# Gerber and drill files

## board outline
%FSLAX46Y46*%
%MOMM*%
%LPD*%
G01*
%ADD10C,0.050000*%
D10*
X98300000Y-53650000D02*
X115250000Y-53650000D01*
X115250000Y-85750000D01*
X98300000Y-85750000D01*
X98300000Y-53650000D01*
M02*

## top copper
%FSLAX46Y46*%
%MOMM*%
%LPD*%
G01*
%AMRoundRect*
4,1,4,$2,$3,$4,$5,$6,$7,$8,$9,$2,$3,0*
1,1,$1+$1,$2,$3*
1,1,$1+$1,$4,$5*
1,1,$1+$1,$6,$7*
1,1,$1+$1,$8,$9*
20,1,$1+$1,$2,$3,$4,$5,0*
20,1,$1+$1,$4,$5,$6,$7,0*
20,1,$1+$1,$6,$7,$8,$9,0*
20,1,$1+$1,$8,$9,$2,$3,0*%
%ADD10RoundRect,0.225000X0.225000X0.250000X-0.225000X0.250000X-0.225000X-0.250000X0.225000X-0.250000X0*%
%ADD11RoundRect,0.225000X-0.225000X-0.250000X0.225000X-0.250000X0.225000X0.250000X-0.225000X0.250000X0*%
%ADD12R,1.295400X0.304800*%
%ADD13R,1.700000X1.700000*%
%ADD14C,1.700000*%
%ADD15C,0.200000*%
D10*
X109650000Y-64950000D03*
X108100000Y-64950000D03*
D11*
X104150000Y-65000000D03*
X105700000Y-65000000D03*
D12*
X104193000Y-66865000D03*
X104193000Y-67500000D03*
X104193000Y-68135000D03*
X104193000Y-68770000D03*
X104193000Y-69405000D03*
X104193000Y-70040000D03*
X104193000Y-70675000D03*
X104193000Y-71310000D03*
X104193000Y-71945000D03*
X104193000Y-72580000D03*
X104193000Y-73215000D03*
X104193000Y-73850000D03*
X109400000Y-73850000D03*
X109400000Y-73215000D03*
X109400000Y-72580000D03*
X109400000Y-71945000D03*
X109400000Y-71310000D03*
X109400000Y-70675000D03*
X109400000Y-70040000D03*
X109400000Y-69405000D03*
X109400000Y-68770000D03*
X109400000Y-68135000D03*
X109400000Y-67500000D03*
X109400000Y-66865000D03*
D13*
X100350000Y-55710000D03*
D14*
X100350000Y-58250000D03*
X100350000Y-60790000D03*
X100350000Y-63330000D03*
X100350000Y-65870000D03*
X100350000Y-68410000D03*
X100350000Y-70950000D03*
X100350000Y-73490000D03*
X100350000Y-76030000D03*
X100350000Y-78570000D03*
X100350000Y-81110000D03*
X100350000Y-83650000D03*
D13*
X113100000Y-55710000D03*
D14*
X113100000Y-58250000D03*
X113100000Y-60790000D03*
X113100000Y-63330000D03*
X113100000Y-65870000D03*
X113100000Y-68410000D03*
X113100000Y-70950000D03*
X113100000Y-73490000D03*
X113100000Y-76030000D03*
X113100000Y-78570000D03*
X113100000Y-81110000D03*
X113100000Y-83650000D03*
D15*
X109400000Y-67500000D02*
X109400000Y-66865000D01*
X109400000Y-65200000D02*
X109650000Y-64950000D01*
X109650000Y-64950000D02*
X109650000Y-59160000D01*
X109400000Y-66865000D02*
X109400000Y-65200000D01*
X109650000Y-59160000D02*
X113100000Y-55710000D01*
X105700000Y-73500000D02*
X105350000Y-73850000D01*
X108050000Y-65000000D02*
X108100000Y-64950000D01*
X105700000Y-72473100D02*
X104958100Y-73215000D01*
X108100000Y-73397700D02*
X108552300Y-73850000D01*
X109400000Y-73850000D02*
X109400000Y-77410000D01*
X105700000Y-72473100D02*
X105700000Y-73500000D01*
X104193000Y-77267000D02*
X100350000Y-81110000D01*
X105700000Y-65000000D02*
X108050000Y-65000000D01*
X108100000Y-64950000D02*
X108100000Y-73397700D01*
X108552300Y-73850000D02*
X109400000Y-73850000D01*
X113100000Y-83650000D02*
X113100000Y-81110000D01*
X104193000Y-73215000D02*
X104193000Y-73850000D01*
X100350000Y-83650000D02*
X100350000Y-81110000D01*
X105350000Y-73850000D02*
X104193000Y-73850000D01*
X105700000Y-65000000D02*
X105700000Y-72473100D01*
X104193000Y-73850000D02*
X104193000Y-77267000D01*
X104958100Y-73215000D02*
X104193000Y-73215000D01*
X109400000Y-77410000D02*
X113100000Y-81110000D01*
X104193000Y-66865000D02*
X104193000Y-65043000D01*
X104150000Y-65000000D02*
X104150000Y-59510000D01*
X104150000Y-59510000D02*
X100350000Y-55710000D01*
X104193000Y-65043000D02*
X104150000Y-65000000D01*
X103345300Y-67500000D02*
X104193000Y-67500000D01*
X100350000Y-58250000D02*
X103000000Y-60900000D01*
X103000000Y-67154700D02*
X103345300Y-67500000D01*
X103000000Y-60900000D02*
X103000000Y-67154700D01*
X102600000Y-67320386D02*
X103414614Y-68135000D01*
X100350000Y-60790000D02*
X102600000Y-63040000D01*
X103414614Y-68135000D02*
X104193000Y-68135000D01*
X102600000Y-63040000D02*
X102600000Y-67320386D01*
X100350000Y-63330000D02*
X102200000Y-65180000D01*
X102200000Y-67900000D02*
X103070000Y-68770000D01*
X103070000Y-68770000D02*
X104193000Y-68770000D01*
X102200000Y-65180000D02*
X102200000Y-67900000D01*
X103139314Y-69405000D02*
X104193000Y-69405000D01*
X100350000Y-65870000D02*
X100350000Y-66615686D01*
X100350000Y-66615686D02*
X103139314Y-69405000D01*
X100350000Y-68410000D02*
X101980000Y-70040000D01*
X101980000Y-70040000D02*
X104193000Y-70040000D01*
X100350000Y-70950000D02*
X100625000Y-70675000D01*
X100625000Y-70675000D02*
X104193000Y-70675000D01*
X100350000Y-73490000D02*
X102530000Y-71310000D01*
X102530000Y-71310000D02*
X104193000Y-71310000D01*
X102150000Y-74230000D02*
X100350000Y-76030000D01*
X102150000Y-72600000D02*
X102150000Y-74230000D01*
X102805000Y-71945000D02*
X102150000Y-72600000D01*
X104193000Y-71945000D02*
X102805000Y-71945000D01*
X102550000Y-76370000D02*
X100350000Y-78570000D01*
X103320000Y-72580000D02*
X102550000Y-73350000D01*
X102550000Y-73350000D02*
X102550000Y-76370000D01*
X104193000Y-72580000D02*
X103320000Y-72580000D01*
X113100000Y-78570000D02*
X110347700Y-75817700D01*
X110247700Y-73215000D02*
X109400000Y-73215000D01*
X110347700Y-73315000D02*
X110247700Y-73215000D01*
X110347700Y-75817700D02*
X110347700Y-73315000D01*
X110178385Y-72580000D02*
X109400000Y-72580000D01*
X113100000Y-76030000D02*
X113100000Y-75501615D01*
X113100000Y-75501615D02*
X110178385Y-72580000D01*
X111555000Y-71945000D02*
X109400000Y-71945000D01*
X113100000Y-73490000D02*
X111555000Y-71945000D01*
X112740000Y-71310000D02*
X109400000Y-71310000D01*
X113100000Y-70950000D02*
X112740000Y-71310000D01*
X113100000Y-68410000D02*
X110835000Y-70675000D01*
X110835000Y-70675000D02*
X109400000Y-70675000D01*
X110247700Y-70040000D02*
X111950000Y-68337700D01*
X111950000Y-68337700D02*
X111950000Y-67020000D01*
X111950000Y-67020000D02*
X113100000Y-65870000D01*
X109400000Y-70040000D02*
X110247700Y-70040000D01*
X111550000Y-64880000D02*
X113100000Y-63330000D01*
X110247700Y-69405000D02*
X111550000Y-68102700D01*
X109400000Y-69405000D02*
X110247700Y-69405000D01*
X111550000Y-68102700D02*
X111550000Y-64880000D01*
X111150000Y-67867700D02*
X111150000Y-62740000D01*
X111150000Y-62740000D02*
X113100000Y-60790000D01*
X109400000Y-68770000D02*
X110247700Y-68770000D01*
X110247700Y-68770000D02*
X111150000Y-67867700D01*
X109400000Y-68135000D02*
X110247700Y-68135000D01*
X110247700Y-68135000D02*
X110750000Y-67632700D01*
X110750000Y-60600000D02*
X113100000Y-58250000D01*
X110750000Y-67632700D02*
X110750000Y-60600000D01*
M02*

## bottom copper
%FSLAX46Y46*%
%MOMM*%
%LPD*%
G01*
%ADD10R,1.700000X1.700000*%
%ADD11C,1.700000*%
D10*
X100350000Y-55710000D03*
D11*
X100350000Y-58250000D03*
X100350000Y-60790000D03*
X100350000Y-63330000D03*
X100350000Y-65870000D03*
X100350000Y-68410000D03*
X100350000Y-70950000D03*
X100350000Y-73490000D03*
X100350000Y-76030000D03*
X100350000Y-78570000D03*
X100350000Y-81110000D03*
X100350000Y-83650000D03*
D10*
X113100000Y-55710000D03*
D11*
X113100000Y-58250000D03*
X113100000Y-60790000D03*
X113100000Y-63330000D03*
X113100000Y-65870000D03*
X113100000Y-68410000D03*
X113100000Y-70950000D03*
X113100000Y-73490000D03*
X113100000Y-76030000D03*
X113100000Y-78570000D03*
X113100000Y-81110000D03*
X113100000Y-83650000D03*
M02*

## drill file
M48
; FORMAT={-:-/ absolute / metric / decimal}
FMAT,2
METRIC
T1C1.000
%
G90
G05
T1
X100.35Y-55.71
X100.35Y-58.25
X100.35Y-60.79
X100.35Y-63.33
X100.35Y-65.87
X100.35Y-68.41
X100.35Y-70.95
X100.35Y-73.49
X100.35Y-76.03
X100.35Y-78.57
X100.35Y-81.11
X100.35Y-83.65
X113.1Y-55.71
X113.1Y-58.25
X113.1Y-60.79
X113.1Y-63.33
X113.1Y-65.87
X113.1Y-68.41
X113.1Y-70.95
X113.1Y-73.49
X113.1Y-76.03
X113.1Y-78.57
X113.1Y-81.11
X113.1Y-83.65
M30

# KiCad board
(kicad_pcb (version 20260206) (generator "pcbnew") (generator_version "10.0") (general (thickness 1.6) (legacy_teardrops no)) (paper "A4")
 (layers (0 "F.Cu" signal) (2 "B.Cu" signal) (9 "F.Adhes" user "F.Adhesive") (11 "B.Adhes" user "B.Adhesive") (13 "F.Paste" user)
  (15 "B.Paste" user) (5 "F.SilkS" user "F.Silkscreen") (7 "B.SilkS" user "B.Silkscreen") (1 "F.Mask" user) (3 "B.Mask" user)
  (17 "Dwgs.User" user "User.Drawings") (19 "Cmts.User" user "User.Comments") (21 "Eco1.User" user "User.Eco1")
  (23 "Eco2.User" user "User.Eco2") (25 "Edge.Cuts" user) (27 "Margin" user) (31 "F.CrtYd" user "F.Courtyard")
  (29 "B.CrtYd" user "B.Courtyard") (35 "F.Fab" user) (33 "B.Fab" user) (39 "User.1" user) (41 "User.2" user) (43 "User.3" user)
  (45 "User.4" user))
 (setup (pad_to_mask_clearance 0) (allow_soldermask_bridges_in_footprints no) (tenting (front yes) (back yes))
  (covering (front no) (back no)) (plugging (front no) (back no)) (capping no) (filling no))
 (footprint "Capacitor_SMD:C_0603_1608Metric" (layer "F.Cu") (at 108.875 64.95 180)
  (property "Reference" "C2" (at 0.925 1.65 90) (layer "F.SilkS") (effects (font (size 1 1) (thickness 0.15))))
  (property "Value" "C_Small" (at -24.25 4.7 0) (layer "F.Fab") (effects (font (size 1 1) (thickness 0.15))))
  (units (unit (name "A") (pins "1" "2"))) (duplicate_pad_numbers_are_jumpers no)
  (pad "1" smd roundrect (at -0.775 0 180) (size 0.9 0.95) (layers "F.Cu" "F.Mask" "F.Paste") (roundrect_rratio 0.25) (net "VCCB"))
  (pad "2" smd roundrect (at 0.775 0 180) (size 0.9 0.95) (layers "F.Cu" "F.Mask" "F.Paste") (roundrect_rratio 0.25) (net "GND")))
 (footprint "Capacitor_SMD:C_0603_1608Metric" (layer "F.Cu") (at 104.925 65)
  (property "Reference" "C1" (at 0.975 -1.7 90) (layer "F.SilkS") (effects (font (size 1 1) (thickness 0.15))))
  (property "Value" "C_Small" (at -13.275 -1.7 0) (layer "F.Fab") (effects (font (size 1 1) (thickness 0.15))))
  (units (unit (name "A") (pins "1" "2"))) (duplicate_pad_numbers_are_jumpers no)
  (pad "1" smd roundrect (at -0.775 0) (size 0.9 0.95) (layers "F.Cu" "F.Mask" "F.Paste") (roundrect_rratio 0.25) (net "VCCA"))
  (pad "2" smd roundrect (at 0.775 0) (size 0.9 0.95) (layers "F.Cu" "F.Mask" "F.Paste") (roundrect_rratio 0.25) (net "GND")))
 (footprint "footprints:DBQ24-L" (layer "F.Cu") (at 106.7965 70.3575)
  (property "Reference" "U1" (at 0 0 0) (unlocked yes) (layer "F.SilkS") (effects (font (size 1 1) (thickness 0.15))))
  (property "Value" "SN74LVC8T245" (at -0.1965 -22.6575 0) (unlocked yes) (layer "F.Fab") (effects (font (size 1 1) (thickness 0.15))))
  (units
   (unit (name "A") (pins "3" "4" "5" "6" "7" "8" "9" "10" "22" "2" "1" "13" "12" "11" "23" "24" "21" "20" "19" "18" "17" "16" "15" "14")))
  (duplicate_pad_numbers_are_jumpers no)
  (pad "1" smd rect (at -2.6035 -3.4925) (size 1.2954 0.3048) (layers "F.Cu" "F.Mask" "F.Paste") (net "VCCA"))
  (pad "2" smd rect (at -2.6035 -2.8575) (size 1.2954 0.3048) (layers "F.Cu" "F.Mask" "F.Paste") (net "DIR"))
  (pad "3" smd rect (at -2.6035 -2.2225) (size 1.2954 0.3048) (layers "F.Cu" "F.Mask" "F.Paste") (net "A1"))
  (pad "4" smd rect (at -2.6035 -1.5875) (size 1.2954 0.3048) (layers "F.Cu" "F.Mask" "F.Paste") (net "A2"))
  (pad "5" smd rect (at -2.6035 -0.9525) (size 1.2954 0.3048) (layers "F.Cu" "F.Mask" "F.Paste") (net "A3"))
  (pad "6" smd rect (at -2.6035 -0.3175) (size 1.2954 0.3048) (layers "F.Cu" "F.Mask" "F.Paste") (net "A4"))
  (pad "7" smd rect (at -2.6035 0.3175) (size 1.2954 0.3048) (layers "F.Cu" "F.Mask" "F.Paste") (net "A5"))
  (pad "8" smd rect (at -2.6035 0.9525) (size 1.2954 0.3048) (layers "F.Cu" "F.Mask" "F.Paste") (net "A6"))
  (pad "9" smd rect (at -2.6035 1.5875) (size 1.2954 0.3048) (layers "F.Cu" "F.Mask" "F.Paste") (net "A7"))
  (pad "10" smd rect (at -2.6035 2.2225) (size 1.2954 0.3048) (layers "F.Cu" "F.Mask" "F.Paste") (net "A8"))
  (pad "11" smd rect (at -2.6035 2.8575) (size 1.2954 0.3048) (layers "F.Cu" "F.Mask" "F.Paste") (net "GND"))
  (pad "12" smd rect (at -2.6035 3.4925) (size 1.2954 0.3048) (layers "F.Cu" "F.Mask" "F.Paste") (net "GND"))
  (pad "13" smd rect (at 2.6035 3.4925) (size 1.2954 0.3048) (layers "F.Cu" "F.Mask" "F.Paste") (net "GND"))
  (pad "14" smd rect (at 2.6035 2.8575) (size 1.2954 0.3048) (layers "F.Cu" "F.Mask" "F.Paste") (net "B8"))
  (pad "15" smd rect (at 2.6035 2.2225) (size 1.2954 0.3048) (layers "F.Cu" "F.Mask" "F.Paste") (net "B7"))
  (pad "16" smd rect (at 2.6035 1.5875) (size 1.2954 0.3048) (layers "F.Cu" "F.Mask" "F.Paste") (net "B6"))
  (pad "17" smd rect (at 2.6035 0.9525) (size 1.2954 0.3048) (layers "F.Cu" "F.Mask" "F.Paste") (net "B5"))
  (pad "18" smd rect (at 2.6035 0.3175) (size 1.2954 0.3048) (layers "F.Cu" "F.Mask" "F.Paste") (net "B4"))
  (pad "19" smd rect (at 2.6035 -0.3175) (size 1.2954 0.3048) (layers "F.Cu" "F.Mask" "F.Paste") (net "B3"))
  (pad "20" smd rect (at 2.6035 -0.9525) (size 1.2954 0.3048) (layers "F.Cu" "F.Mask" "F.Paste") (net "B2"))
  (pad "21" smd rect (at 2.6035 -1.5875) (size 1.2954 0.3048) (layers "F.Cu" "F.Mask" "F.Paste") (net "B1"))
  (pad "22" smd rect (at 2.6035 -2.2225) (size 1.2954 0.3048) (layers "F.Cu" "F.Mask" "F.Paste") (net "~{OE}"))
  (pad "23" smd rect (at 2.6035 -2.8575) (size 1.2954 0.3048) (layers "F.Cu" "F.Mask" "F.Paste") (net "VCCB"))
  (pad "24" smd rect (at 2.6035 -3.4925) (size 1.2954 0.3048) (layers "F.Cu" "F.Mask" "F.Paste") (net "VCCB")))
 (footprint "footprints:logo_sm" (layer "F.Cu") (at 106.8 80.325)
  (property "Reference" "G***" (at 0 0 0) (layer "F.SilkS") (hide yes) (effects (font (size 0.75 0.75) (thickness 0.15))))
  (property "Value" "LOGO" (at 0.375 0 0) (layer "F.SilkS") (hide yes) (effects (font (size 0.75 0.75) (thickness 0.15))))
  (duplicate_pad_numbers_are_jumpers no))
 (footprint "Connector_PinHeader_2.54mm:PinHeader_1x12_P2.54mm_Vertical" (layer "B.Cu") (at 100.35 55.71 180)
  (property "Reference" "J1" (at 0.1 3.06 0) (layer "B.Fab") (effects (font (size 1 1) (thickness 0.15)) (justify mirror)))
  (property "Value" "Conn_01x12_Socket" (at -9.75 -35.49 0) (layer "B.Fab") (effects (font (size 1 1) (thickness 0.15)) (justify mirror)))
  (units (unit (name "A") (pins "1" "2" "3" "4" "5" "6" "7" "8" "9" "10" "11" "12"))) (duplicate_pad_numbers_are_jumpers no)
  (pad "1" thru_hole rect (at 0 0 180) (size 1.7 1.7) (drill 1) (layers "*.Cu" "*.Mask") (remove_unused_layers no) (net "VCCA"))
  (pad "2" thru_hole circle (at 0 -2.54 180) (size 1.7 1.7) (drill 1) (layers "*.Cu" "*.Mask") (remove_unused_layers no) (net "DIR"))
  (pad "3" thru_hole circle (at 0 -5.08 180) (size 1.7 1.7) (drill 1) (layers "*.Cu" "*.Mask") (remove_unused_layers no) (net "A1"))
  (pad "4" thru_hole circle (at 0 -7.62 180) (size 1.7 1.7) (drill 1) (layers "*.Cu" "*.Mask") (remove_unused_layers no) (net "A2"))
  (pad "5" thru_hole circle (at 0 -10.16 180) (size 1.7 1.7) (drill 1) (layers "*.Cu" "*.Mask") (remove_unused_layers no) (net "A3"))
  (pad "6" thru_hole circle (at 0 -12.7 180) (size 1.7 1.7) (drill 1) (layers "*.Cu" "*.Mask") (remove_unused_layers no) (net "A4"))
  (pad "7" thru_hole circle (at 0 -15.24 180) (size 1.7 1.7) (drill 1) (layers "*.Cu" "*.Mask") (remove_unused_layers no) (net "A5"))
  (pad "8" thru_hole circle (at 0 -17.78 180) (size 1.7 1.7) (drill 1) (layers "*.Cu" "*.Mask") (remove_unused_layers no) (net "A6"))
  (pad "9" thru_hole circle (at 0 -20.32 180) (size 1.7 1.7) (drill 1) (layers "*.Cu" "*.Mask") (remove_unused_layers no) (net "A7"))
  (pad "10" thru_hole circle (at 0 -22.86 180) (size 1.7 1.7) (drill 1) (layers "*.Cu" "*.Mask") (remove_unused_layers no) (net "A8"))
  (pad "11" thru_hole circle (at 0 -25.4 180) (size 1.7 1.7) (drill 1) (layers "*.Cu" "*.Mask") (remove_unused_layers no) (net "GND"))
  (pad "12" thru_hole circle (at 0 -27.94 180) (size 1.7 1.7) (drill 1) (layers "*.Cu" "*.Mask") (remove_unused_layers no) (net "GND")))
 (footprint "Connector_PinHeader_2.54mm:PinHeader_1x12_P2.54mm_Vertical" (layer "B.Cu") (at 113.1 55.71 180)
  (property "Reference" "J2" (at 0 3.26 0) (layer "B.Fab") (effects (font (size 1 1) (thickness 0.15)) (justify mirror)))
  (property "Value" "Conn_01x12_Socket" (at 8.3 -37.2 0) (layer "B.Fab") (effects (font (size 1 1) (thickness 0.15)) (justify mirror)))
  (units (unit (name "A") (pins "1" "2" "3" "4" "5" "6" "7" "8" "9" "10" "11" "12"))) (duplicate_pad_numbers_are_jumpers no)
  (pad "1" thru_hole rect (at 0 0 180) (size 1.7 1.7) (drill 1) (layers "*.Cu" "*.Mask") (remove_unused_layers no) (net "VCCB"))
  (pad "2" thru_hole circle (at 0 -2.54 180) (size 1.7 1.7) (drill 1) (layers "*.Cu" "*.Mask") (remove_unused_layers no) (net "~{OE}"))
  (pad "3" thru_hole circle (at 0 -5.08 180) (size 1.7 1.7) (drill 1) (layers "*.Cu" "*.Mask") (remove_unused_layers no) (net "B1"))
  (pad "4" thru_hole circle (at 0 -7.62 180) (size 1.7 1.7) (drill 1) (layers "*.Cu" "*.Mask") (remove_unused_layers no) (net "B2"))
  (pad "5" thru_hole circle (at 0 -10.16 180) (size 1.7 1.7) (drill 1) (layers "*.Cu" "*.Mask") (remove_unused_layers no) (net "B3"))
  (pad "6" thru_hole circle (at 0 -12.7 180) (size 1.7 1.7) (drill 1) (layers "*.Cu" "*.Mask") (remove_unused_layers no) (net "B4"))
  (pad "7" thru_hole circle (at 0 -15.24 180) (size 1.7 1.7) (drill 1) (layers "*.Cu" "*.Mask") (remove_unused_layers no) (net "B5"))
  (pad "8" thru_hole circle (at 0 -17.78 180) (size 1.7 1.7) (drill 1) (layers "*.Cu" "*.Mask") (remove_unused_layers no) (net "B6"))
  (pad "9" thru_hole circle (at 0 -20.32 180) (size 1.7 1.7) (drill 1) (layers "*.Cu" "*.Mask") (remove_unused_layers no) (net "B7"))
  (pad "10" thru_hole circle (at 0 -22.86 180) (size 1.7 1.7) (drill 1) (layers "*.Cu" "*.Mask") (remove_unused_layers no) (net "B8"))
  (pad "11" thru_hole circle (at 0 -25.4 180) (size 1.7 1.7) (drill 1) (layers "*.Cu" "*.Mask") (remove_unused_layers no) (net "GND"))
  (pad "12" thru_hole circle (at 0 -27.94 180) (size 1.7 1.7) (drill 1) (layers "*.Cu" "*.Mask") (remove_unused_layers no) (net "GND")))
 (gr_rect (start 98.3 53.65) (end 115.25 85.75) (stroke (width 0.05) (type default)) (fill no) (layer "Edge.Cuts"))
 (segment (start 109.4 67.5) (end 109.4 66.865) (width 0.2) (layer "F.Cu") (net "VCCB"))
 (segment (start 109.4 65.2) (end 109.65 64.95) (width 0.2) (layer "F.Cu") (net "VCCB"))
 (segment (start 109.65 64.95) (end 109.65 59.16) (width 0.2) (layer "F.Cu") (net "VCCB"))
 (segment (start 109.4 66.865) (end 109.4 65.2) (width 0.2) (layer "F.Cu") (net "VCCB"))
 (segment (start 109.65 59.16) (end 113.1 55.71) (width 0.2) (layer "F.Cu") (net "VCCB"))
 (segment (start 105.7 73.5) (end 105.35 73.85) (width 0.2) (layer "F.Cu") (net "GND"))
 (segment (start 108.05 65) (end 108.1 64.95) (width 0.2) (layer "F.Cu") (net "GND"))
 (segment (start 105.7 72.4731) (end 104.9581 73.215) (width 0.2) (layer "F.Cu") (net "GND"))
 (segment (start 108.1 73.3977) (end 108.5523 73.85) (width 0.2) (layer "F.Cu") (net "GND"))
 (segment (start 109.4 73.85) (end 109.4 77.41) (width 0.2) (layer "F.Cu") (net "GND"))
 (segment (start 105.7 72.4731) (end 105.7 73.5) (width 0.2) (layer "F.Cu") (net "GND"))
 (segment (start 104.193 77.267) (end 100.35 81.11) (width 0.2) (layer "F.Cu") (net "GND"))
 (segment (start 105.7 65) (end 108.05 65) (width 0.2) (layer "F.Cu") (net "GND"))
 (segment (start 108.1 64.95) (end 108.1 73.3977) (width 0.2) (layer "F.Cu") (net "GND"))
 (segment (start 108.5523 73.85) (end 109.4 73.85) (width 0.2) (layer "F.Cu") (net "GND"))
 (segment (start 113.1 83.65) (end 113.1 81.11) (width 0.2) (layer "F.Cu") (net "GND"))
 (segment (start 104.193 73.215) (end 104.193 73.85) (width 0.2) (layer "F.Cu") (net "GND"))
 (segment (start 100.35 83.65) (end 100.35 81.11) (width 0.2) (layer "F.Cu") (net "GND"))
 (segment (start 105.35 73.85) (end 104.193 73.85) (width 0.2) (layer "F.Cu") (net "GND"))
 (segment (start 105.7 65) (end 105.7 72.4731) (width 0.2) (layer "F.Cu") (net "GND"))
 (segment (start 104.193 73.85) (end 104.193 77.267) (width 0.2) (layer "F.Cu") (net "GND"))
 (segment (start 104.9581 73.215) (end 104.193 73.215) (width 0.2) (layer "F.Cu") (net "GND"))
 (segment (start 109.4 77.41) (end 113.1 81.11) (width 0.2) (layer "F.Cu") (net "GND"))
 (segment (start 104.193 66.865) (end 104.193 65.043) (width 0.2) (layer "F.Cu") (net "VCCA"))
 (segment (start 104.15 65) (end 104.15 59.51) (width 0.2) (layer "F.Cu") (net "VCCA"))
 (segment (start 104.15 59.51) (end 100.35 55.71) (width 0.2) (layer "F.Cu") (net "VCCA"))
 (segment (start 104.193 65.043) (end 104.15 65) (width 0.2) (layer "F.Cu") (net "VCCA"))
 (segment (start 103.3453 67.5) (end 104.193 67.5) (width 0.2) (layer "F.Cu") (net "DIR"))
 (segment (start 100.35 58.25) (end 103 60.9) (width 0.2) (layer "F.Cu") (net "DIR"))
 (segment (start 103 67.1547) (end 103.3453 67.5) (width 0.2) (layer "F.Cu") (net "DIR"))
 (segment (start 103 60.9) (end 103 67.1547) (width 0.2) (layer "F.Cu") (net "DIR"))
 (segment (start 102.6 67.320386) (end 103.414614 68.135) (width 0.2) (layer "F.Cu") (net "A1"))
 (segment (start 100.35 60.79) (end 102.6 63.04) (width 0.2) (layer "F.Cu") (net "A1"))
 (segment (start 103.414614 68.135) (end 104.193 68.135) (width 0.2) (layer "F.Cu") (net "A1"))
 (segment (start 102.6 63.04) (end 102.6 67.320386) (width 0.2) (layer "F.Cu") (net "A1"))
 (segment (start 100.35 63.33) (end 102.2 65.18) (width 0.2) (layer "F.Cu") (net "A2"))
 (segment (start 102.2 67.9) (end 103.07 68.77) (width 0.2) (layer "F.Cu") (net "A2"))
 (segment (start 103.07 68.77) (end 104.193 68.77) (width 0.2) (layer "F.Cu") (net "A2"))
 (segment (start 102.2 65.18) (end 102.2 67.9) (width 0.2) (layer "F.Cu") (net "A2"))
 (segment (start 103.139314 69.405) (end 104.193 69.405) (width 0.2) (layer "F.Cu") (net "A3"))
 (segment (start 100.35 65.87) (end 100.35 66.615686) (width 0.2) (layer "F.Cu") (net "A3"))
 (segment (start 100.35 66.615686) (end 103.139314 69.405) (width 0.2) (layer "F.Cu") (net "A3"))
 (segment (start 100.35 68.41) (end 101.98 70.04) (width 0.2) (layer "F.Cu") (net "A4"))
 (segment (start 101.98 70.04) (end 104.193 70.04) (width 0.2) (layer "F.Cu") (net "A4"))
 (segment (start 100.35 70.95) (end 100.625 70.675) (width 0.2) (layer "F.Cu") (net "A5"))
 (segment (start 100.625 70.675) (end 104.193 70.675) (width 0.2) (layer "F.Cu") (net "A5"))
 (segment (start 100.35 73.49) (end 102.53 71.31) (width 0.2) (layer "F.Cu") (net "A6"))
 (segment (start 102.53 71.31) (end 104.193 71.31) (width 0.2) (layer "F.Cu") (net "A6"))
 (segment (start 102.15 74.23) (end 100.35 76.03) (width 0.2) (layer "F.Cu") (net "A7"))
 (segment (start 102.15 72.6) (end 102.15 74.23) (width 0.2) (layer "F.Cu") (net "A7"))
 (segment (start 102.805 71.945) (end 102.15 72.6) (width 0.2) (layer "F.Cu") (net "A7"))
 (segment (start 104.193 71.945) (end 102.805 71.945) (width 0.2) (layer "F.Cu") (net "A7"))
 (segment (start 102.55 76.37) (end 100.35 78.57) (width 0.2) (layer "F.Cu") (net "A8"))
 (segment (start 103.32 72.58) (end 102.55 73.35) (width 0.2) (layer "F.Cu") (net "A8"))
 (segment (start 102.55 73.35) (end 102.55 76.37) (width 0.2) (layer "F.Cu") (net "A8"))
 (segment (start 104.193 72.58) (end 103.32 72.58) (width 0.2) (layer "F.Cu") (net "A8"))
 (segment (start 113.1 78.57) (end 110.3477 75.8177) (width 0.2) (layer "F.Cu") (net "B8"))
 (segment (start 110.2477 73.215) (end 109.4 73.215) (width 0.2) (layer "F.Cu") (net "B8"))
 (segment (start 110.3477 73.315) (end 110.2477 73.215) (width 0.2) (layer "F.Cu") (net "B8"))
 (segment (start 110.3477 75.8177) (end 110.3477 73.315) (width 0.2) (layer "F.Cu") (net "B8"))
 (segment (start 110.178385 72.58) (end 109.4 72.58) (width 0.2) (layer "F.Cu") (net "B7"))
 (segment (start 113.1 76.03) (end 113.1 75.501615) (width 0.2) (layer "F.Cu") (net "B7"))
 (segment (start 113.1 75.501615) (end 110.178385 72.58) (width 0.2) (layer "F.Cu") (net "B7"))
 (segment (start 111.555 71.945) (end 109.4 71.945) (width 0.2) (layer "F.Cu") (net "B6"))
 (segment (start 113.1 73.49) (end 111.555 71.945) (width 0.2) (layer "F.Cu") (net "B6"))
 (segment (start 112.74 71.31) (end 109.4 71.31) (width 0.2) (layer "F.Cu") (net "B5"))
 (segment (start 113.1 70.95) (end 112.74 71.31) (width 0.2) (layer "F.Cu") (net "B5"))
 (segment (start 113.1 68.41) (end 110.835 70.675) (width 0.2) (layer "F.Cu") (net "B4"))
 (segment (start 110.835 70.675) (end 109.4 70.675) (width 0.2) (layer "F.Cu") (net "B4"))
 (segment (start 110.2477 70.04) (end 111.95 68.3377) (width 0.2) (layer "F.Cu") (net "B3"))
 (segment (start 111.95 68.3377) (end 111.95 67.02) (width 0.2) (layer "F.Cu") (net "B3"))
 (segment (start 111.95 67.02) (end 113.1 65.87) (width 0.2) (layer "F.Cu") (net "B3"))
 (segment (start 109.4 70.04) (end 110.2477 70.04) (width 0.2) (layer "F.Cu") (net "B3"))
 (segment (start 111.55 64.88) (end 113.1 63.33) (width 0.2) (layer "F.Cu") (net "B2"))
 (segment (start 110.2477 69.405) (end 111.55 68.1027) (width 0.2) (layer "F.Cu") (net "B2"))
 (segment (start 109.4 69.405) (end 110.2477 69.405) (width 0.2) (layer "F.Cu") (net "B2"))
 (segment (start 111.55 68.1027) (end 111.55 64.88) (width 0.2) (layer "F.Cu") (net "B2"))
 (segment (start 111.15 67.8677) (end 111.15 62.74) (width 0.2) (layer "F.Cu") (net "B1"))
 (segment (start 111.15 62.74) (end 113.1 60.79) (width 0.2) (layer "F.Cu") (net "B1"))
 (segment (start 109.4 68.77) (end 110.2477 68.77) (width 0.2) (layer "F.Cu") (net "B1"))
 (segment (start 110.2477 68.77) (end 111.15 67.8677) (width 0.2) (layer "F.Cu") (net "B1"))
 (segment (start 109.4 68.135) (end 110.2477 68.135) (width 0.2) (layer "F.Cu") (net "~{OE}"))
 (segment (start 110.2477 68.135) (end 110.75 67.6327) (width 0.2) (layer "F.Cu") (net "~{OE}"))
 (segment (start 110.75 60.6) (end 113.1 58.25) (width 0.2) (layer "F.Cu") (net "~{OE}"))
 (segment (start 110.75 67.6327) (end 110.75 60.6) (width 0.2) (layer "F.Cu") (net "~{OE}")))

